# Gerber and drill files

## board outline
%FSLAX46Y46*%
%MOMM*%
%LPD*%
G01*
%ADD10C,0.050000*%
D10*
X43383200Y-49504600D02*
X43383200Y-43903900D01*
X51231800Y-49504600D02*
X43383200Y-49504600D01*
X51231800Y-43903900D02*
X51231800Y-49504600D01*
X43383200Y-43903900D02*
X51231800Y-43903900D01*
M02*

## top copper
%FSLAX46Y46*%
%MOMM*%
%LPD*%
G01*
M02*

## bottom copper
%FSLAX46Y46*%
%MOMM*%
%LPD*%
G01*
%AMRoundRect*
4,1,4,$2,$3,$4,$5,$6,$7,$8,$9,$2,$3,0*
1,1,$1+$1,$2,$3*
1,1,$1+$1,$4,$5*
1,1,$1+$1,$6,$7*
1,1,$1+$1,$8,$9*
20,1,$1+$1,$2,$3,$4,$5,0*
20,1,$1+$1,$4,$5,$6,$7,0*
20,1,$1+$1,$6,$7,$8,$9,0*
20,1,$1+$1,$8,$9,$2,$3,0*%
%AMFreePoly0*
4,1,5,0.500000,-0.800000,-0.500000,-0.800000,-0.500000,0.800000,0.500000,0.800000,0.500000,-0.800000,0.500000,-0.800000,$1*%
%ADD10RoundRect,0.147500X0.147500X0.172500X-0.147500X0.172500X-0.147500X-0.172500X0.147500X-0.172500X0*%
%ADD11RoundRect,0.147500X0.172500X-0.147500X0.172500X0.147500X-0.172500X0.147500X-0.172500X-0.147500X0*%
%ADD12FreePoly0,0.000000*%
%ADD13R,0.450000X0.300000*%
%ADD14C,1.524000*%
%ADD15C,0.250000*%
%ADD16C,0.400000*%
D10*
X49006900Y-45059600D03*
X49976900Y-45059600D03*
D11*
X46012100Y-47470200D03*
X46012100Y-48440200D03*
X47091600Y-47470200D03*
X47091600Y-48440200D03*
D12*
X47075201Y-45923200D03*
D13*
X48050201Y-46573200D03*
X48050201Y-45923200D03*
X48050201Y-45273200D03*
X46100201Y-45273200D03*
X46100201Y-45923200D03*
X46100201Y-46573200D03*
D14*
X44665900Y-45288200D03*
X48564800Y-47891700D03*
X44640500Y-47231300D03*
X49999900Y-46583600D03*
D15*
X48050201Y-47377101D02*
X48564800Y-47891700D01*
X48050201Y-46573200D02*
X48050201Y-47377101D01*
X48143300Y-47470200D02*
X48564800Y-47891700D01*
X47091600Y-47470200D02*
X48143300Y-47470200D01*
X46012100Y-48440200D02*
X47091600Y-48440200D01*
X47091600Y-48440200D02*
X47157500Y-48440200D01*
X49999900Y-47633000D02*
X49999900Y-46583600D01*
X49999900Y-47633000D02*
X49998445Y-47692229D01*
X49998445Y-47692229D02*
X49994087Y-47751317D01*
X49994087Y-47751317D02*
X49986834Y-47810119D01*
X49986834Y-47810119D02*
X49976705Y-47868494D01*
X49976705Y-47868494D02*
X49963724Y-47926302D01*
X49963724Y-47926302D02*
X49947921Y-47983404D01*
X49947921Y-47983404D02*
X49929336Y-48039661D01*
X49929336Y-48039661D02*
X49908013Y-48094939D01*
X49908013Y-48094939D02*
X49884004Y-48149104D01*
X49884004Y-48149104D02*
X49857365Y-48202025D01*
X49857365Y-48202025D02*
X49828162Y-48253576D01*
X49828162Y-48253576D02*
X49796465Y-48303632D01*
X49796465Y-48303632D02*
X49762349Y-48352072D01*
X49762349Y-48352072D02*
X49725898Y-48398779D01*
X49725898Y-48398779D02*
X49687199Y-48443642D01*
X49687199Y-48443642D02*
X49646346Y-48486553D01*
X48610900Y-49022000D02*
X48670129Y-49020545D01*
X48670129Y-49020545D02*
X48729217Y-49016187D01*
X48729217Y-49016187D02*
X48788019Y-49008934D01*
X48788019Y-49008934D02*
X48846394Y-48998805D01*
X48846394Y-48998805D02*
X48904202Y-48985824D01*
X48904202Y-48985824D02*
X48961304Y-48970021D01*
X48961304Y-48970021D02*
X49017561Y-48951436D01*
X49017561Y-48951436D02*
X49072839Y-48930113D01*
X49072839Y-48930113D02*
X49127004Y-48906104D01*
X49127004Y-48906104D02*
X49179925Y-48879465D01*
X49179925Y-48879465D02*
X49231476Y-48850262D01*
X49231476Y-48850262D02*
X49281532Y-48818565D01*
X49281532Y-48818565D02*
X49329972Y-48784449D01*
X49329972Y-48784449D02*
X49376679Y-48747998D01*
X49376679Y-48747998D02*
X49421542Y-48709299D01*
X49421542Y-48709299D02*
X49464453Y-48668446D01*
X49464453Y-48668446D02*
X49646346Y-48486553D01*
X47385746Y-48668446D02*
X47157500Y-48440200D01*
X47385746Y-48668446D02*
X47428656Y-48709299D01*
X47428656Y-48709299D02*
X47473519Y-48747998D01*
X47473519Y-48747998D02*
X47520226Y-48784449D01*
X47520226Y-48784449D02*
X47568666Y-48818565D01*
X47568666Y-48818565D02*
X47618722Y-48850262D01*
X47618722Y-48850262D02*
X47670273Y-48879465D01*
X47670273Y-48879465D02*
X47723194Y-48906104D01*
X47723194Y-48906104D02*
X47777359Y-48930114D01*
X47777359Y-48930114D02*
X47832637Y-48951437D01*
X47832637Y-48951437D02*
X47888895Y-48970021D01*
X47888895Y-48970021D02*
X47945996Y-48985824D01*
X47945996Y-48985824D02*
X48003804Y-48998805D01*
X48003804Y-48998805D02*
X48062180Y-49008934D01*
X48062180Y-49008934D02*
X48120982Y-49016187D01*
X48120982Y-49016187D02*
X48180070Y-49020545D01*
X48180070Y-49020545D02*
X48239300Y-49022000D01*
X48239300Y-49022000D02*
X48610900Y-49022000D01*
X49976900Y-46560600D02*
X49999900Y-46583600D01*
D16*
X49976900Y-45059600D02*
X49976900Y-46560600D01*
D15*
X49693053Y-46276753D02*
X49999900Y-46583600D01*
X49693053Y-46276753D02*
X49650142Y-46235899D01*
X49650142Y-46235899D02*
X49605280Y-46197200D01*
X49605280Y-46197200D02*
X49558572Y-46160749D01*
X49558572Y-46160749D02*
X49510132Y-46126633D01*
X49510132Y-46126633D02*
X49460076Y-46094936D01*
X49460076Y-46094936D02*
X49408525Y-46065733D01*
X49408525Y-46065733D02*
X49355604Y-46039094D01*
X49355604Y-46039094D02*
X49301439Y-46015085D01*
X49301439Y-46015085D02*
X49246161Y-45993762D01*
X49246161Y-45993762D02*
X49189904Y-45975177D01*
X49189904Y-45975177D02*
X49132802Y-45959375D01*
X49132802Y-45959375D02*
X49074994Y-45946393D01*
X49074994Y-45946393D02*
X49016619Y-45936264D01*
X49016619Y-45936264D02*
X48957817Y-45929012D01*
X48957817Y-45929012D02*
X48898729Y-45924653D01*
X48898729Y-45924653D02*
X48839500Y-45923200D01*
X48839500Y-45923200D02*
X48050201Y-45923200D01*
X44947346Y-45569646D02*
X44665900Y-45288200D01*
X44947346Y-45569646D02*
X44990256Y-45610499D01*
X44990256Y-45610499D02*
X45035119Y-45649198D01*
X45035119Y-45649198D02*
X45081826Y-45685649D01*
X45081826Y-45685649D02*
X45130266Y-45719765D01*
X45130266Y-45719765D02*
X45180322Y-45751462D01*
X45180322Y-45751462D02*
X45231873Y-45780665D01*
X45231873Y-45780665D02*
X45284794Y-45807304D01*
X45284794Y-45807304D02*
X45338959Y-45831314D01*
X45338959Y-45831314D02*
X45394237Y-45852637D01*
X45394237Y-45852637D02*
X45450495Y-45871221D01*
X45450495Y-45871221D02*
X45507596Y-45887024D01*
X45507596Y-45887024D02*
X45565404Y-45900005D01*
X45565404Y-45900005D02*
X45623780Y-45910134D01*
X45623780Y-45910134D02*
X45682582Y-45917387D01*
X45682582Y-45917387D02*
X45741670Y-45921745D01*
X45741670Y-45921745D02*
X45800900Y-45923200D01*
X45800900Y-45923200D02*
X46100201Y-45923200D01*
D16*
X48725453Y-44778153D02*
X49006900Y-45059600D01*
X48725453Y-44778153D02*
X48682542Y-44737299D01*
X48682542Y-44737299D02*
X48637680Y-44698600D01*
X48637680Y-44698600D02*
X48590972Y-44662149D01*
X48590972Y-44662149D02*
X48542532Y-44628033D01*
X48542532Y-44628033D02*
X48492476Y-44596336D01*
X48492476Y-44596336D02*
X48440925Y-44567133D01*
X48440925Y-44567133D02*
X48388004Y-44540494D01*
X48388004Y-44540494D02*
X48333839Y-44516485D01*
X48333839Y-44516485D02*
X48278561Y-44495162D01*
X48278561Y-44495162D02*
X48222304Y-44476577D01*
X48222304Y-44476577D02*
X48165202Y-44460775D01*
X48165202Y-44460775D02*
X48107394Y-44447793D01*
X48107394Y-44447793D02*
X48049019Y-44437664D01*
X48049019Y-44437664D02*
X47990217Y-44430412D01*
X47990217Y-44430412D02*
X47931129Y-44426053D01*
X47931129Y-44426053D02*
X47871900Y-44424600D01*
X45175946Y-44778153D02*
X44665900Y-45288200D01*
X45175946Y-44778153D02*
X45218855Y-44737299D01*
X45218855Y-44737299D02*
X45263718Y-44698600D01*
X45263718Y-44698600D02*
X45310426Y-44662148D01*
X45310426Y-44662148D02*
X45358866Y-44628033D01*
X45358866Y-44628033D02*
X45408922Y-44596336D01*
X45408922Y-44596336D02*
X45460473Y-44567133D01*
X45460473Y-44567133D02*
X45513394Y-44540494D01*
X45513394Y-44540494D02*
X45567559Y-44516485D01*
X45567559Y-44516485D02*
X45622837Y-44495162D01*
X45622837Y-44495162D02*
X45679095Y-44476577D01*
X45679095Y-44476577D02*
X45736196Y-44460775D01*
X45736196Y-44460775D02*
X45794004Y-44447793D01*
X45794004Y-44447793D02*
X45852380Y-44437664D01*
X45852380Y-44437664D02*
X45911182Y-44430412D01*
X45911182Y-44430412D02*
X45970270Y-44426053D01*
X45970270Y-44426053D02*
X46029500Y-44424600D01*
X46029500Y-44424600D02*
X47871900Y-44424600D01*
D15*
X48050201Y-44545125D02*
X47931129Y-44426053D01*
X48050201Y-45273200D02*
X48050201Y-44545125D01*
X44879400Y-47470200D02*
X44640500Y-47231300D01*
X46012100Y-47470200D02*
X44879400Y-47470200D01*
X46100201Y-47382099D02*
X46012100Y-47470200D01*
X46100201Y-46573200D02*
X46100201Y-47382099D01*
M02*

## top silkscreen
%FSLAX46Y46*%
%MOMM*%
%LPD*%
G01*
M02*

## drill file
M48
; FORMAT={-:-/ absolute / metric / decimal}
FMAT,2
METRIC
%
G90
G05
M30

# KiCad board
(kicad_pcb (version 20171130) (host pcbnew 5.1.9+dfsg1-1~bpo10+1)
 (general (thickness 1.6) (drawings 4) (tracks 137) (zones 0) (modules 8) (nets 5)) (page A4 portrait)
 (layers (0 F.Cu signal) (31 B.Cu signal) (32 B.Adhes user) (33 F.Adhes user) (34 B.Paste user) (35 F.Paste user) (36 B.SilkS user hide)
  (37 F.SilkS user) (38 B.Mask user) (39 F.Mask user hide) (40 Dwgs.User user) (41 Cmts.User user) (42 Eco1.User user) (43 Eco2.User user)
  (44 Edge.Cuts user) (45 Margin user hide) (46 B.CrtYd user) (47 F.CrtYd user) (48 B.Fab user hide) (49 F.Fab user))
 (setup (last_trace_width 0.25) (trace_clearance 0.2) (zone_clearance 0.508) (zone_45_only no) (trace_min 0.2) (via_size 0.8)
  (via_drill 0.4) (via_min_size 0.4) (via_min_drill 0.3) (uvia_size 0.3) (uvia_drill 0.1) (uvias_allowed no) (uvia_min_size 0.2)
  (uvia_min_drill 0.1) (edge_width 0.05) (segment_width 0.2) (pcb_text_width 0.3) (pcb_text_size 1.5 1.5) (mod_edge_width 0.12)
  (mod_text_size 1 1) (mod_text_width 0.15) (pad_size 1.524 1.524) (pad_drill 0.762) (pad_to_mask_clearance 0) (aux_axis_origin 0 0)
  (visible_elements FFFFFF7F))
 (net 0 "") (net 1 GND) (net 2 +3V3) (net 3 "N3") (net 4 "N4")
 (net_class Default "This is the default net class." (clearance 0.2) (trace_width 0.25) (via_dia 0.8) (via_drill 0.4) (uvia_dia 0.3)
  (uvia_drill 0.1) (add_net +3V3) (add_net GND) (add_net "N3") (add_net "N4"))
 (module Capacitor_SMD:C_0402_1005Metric (layer B.Cu) (at 49.4919 45.0596 180)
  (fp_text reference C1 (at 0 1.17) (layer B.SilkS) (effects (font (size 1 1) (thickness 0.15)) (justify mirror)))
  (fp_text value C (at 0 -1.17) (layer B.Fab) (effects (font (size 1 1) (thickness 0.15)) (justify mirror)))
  (pad 2 smd roundrect (at 0.485 0 180) (size 0.59 0.64) (layers B.Cu B.Paste B.Mask) (roundrect_rratio 0.25) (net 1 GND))
  (pad 1 smd roundrect (at -0.485 0 180) (size 0.59 0.64) (layers B.Cu B.Paste B.Mask) (roundrect_rratio 0.25) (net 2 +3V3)))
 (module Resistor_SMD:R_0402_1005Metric (layer B.Cu) (at 46.0121 47.9552 90)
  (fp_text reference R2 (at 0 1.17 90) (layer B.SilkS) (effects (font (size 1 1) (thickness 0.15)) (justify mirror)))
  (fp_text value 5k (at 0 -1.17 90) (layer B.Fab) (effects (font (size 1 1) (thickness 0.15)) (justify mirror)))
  (pad 2 smd roundrect (at 0.485 0 90) (size 0.59 0.64) (layers B.Cu B.Paste B.Mask) (roundrect_rratio 0.25) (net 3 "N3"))
  (pad 1 smd roundrect (at -0.485 0 90) (size 0.59 0.64) (layers B.Cu B.Paste B.Mask) (roundrect_rratio 0.25) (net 2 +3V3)))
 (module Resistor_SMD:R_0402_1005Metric (layer B.Cu) (at 47.0916 47.9552 90)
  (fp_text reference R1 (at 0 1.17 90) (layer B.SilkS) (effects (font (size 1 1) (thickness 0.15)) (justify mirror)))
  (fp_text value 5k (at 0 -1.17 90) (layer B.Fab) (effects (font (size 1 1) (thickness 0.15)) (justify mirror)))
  (pad 2 smd roundrect (at 0.485 0 90) (size 0.59 0.64) (layers B.Cu B.Paste B.Mask) (roundrect_rratio 0.25) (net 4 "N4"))
  (pad 1 smd roundrect (at -0.485 0 90) (size 0.59 0.64) (layers B.Cu B.Paste B.Mask) (roundrect_rratio 0.25) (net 2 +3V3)))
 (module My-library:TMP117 (layer B.Cu) (at 47.075201 45.9232)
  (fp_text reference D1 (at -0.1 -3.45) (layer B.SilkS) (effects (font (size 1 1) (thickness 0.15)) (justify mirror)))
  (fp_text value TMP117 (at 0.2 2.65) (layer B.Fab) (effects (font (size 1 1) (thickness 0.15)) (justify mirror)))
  (pad 7 smd custom (at 0 0) (size 1 1.6) (layers B.Cu B.Paste B.Mask) (zone_connect 0) (options (clearance outline) (anchor rect))
   (primitives))
  (pad 6 smd rect (at 0.975 0.65) (size 0.45 0.3) (layers B.Cu B.Paste B.Mask) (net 4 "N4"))
  (pad 5 smd rect (at 0.975 0) (size 0.45 0.3) (layers B.Cu B.Paste B.Mask) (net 2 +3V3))
  (pad 4 smd rect (at 0.975 -0.65) (size 0.45 0.3) (layers B.Cu B.Paste B.Mask) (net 1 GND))
  (pad 3 smd rect (at -0.975 -0.65) (size 0.45 0.3) (layers B.Cu B.Paste B.Mask))
  (pad 2 smd rect (at -0.975 0) (size 0.45 0.3) (layers B.Cu B.Paste B.Mask) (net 1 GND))
  (pad 1 smd rect (at -0.975 0.65) (size 0.45 0.3) (layers B.Cu B.Paste B.Mask) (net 3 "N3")))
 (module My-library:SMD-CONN (layer B.Cu) (at 44.6659 45.2882)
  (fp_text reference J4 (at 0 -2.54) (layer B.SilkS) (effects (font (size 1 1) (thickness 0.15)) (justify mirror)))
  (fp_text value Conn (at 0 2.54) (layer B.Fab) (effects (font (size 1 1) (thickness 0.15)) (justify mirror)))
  (pad 1 smd circle (at 0 0) (size 1.524 1.524) (layers B.Cu B.Paste B.Mask) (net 1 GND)))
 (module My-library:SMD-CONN (layer B.Cu) (at 48.5648 47.8917)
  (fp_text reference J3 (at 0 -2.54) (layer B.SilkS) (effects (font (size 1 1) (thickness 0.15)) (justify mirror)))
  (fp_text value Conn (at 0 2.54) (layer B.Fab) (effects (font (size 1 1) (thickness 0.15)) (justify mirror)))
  (pad 1 smd circle (at 0 0) (size 1.524 1.524) (layers B.Cu B.Paste B.Mask) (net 4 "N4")))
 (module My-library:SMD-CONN (layer B.Cu) (at 44.6405 47.2313)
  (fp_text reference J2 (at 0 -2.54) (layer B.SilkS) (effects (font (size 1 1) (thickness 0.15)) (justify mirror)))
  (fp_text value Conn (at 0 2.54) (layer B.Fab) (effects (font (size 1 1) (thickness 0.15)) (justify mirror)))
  (pad 1 smd circle (at 0 0) (size 1.524 1.524) (layers B.Cu B.Paste B.Mask) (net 3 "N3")))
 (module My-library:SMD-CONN (layer B.Cu) (at 49.9999 46.5836)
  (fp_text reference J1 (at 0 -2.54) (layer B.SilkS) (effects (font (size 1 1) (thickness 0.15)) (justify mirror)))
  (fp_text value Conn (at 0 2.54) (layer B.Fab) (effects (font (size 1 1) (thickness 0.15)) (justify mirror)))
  (pad 1 smd circle (at 0 0) (size 1.524 1.524) (layers B.Cu B.Paste B.Mask) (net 2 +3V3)))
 (gr_line (start 43.3832 49.5046) (end 43.3832 43.9039) (layer Edge.Cuts) (width 0.05))
 (gr_line (start 51.2318 49.5046) (end 43.3832 49.5046) (layer Edge.Cuts) (width 0.05))
 (gr_line (start 51.2318 43.9039) (end 51.2318 49.5046) (layer Edge.Cuts) (width 0.05))
 (gr_line (start 43.3832 43.9039) (end 51.2318 43.9039) (layer Edge.Cuts) (width 0.05))
 (segment (start 48.050201 47.377101) (end 48.5648 47.8917) (width 0.25) (layer B.Cu) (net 4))
 (segment (start 48.050201 46.5732) (end 48.050201 47.377101) (width 0.25) (layer B.Cu) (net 4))
 (segment (start 48.1433 47.4702) (end 48.5648 47.8917) (width 0.25) (layer B.Cu) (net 4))
 (segment (start 47.0916 47.4702) (end 48.1433 47.4702) (width 0.25) (layer B.Cu) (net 4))
 (segment (start 46.0121 48.4402) (end 47.0916 48.4402) (width 0.25) (layer B.Cu) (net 2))
 (segment (start 47.0916 48.4402) (end 47.1575 48.4402) (width 0.25) (layer B.Cu) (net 2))
 (segment (start 49.9999 47.633) (end 49.9999 46.5836) (width 0.25) (layer B.Cu) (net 2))
 (segment (start 49.9999 47.633) (end 49.998445 47.692229) (width 0.25) (layer B.Cu) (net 2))
 (segment (start 49.998445 47.692229) (end 49.994087 47.751317) (width 0.25) (layer B.Cu) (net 2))
 (segment (start 49.994087 47.751317) (end 49.986834 47.810119) (width 0.25) (layer B.Cu) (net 2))
 (segment (start 49.986834 47.810119) (end 49.976705 47.868494) (width 0.25) (layer B.Cu) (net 2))
 (segment (start 49.976705 47.868494) (end 49.963724 47.926302) (width 0.25) (layer B.Cu) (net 2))
 (segment (start 49.963724 47.926302) (end 49.947921 47.983404) (width 0.25) (layer B.Cu) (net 2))
 (segment (start 49.947921 47.983404) (end 49.929336 48.039661) (width 0.25) (layer B.Cu) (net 2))
 (segment (start 49.929336 48.039661) (end 49.908013 48.094939) (width 0.25) (layer B.Cu) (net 2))
 (segment (start 49.908013 48.094939) (end 49.884004 48.149104) (width 0.25) (layer B.Cu) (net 2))
 (segment (start 49.884004 48.149104) (end 49.857365 48.202025) (width 0.25) (layer B.Cu) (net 2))
 (segment (start 49.857365 48.202025) (end 49.828162 48.253576) (width 0.25) (layer B.Cu) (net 2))
 (segment (start 49.828162 48.253576) (end 49.796465 48.303632) (width 0.25) (layer B.Cu) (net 2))
 (segment (start 49.796465 48.303632) (end 49.762349 48.352072) (width 0.25) (layer B.Cu) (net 2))
 (segment (start 49.762349 48.352072) (end 49.725898 48.398779) (width 0.25) (layer B.Cu) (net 2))
 (segment (start 49.725898 48.398779) (end 49.687199 48.443642) (width 0.25) (layer B.Cu) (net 2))
 (segment (start 49.687199 48.443642) (end 49.646346 48.486553) (width 0.25) (layer B.Cu) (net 2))
 (segment (start 48.6109 49.022) (end 48.670129 49.020545) (width 0.25) (layer B.Cu) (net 2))
 (segment (start 48.670129 49.020545) (end 48.729217 49.016187) (width 0.25) (layer B.Cu) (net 2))
 (segment (start 48.729217 49.016187) (end 48.788019 49.008934) (width 0.25) (layer B.Cu) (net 2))
 (segment (start 48.788019 49.008934) (end 48.846394 48.998805) (width 0.25) (layer B.Cu) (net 2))
 (segment (start 48.846394 48.998805) (end 48.904202 48.985824) (width 0.25) (layer B.Cu) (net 2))
 (segment (start 48.904202 48.985824) (end 48.961304 48.970021) (width 0.25) (layer B.Cu) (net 2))
 (segment (start 48.961304 48.970021) (end 49.017561 48.951436) (width 0.25) (layer B.Cu) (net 2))
 (segment (start 49.017561 48.951436) (end 49.072839 48.930113) (width 0.25) (layer B.Cu) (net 2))
 (segment (start 49.072839 48.930113) (end 49.127004 48.906104) (width 0.25) (layer B.Cu) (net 2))
 (segment (start 49.127004 48.906104) (end 49.179925 48.879465) (width 0.25) (layer B.Cu) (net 2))
 (segment (start 49.179925 48.879465) (end 49.231476 48.850262) (width 0.25) (layer B.Cu) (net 2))
 (segment (start 49.231476 48.850262) (end 49.281532 48.818565) (width 0.25) (layer B.Cu) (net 2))
 (segment (start 49.281532 48.818565) (end 49.329972 48.784449) (width 0.25) (layer B.Cu) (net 2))
 (segment (start 49.329972 48.784449) (end 49.376679 48.747998) (width 0.25) (layer B.Cu) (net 2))
 (segment (start 49.376679 48.747998) (end 49.421542 48.709299) (width 0.25) (layer B.Cu) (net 2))
 (segment (start 49.421542 48.709299) (end 49.464453 48.668446) (width 0.25) (layer B.Cu) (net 2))
 (segment (start 49.464453 48.668446) (end 49.646346 48.486553) (width 0.25) (layer B.Cu) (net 2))
 (segment (start 47.385746 48.668446) (end 47.1575 48.4402) (width 0.25) (layer B.Cu) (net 2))
 (segment (start 47.385746 48.668446) (end 47.428656 48.709299) (width 0.25) (layer B.Cu) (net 2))
 (segment (start 47.428656 48.709299) (end 47.473519 48.747998) (width 0.25) (layer B.Cu) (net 2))
 (segment (start 47.473519 48.747998) (end 47.520226 48.784449) (width 0.25) (layer B.Cu) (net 2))
 (segment (start 47.520226 48.784449) (end 47.568666 48.818565) (width 0.25) (layer B.Cu) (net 2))
 (segment (start 47.568666 48.818565) (end 47.618722 48.850262) (width 0.25) (layer B.Cu) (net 2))
 (segment (start 47.618722 48.850262) (end 47.670273 48.879465) (width 0.25) (layer B.Cu) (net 2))
 (segment (start 47.670273 48.879465) (end 47.723194 48.906104) (width 0.25) (layer B.Cu) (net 2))
 (segment (start 47.723194 48.906104) (end 47.777359 48.930114) (width 0.25) (layer B.Cu) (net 2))
 (segment (start 47.777359 48.930114) (end 47.832637 48.951437) (width 0.25) (layer B.Cu) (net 2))
 (segment (start 47.832637 48.951437) (end 47.888895 48.970021) (width 0.25) (layer B.Cu) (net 2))
 (segment (start 47.888895 48.970021) (end 47.945996 48.985824) (width 0.25) (layer B.Cu) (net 2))
 (segment (start 47.945996 48.985824) (end 48.003804 48.998805) (width 0.25) (layer B.Cu) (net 2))
 (segment (start 48.003804 48.998805) (end 48.06218 49.008934) (width 0.25) (layer B.Cu) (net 2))
 (segment (start 48.06218 49.008934) (end 48.120982 49.016187) (width 0.25) (layer B.Cu) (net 2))
 (segment (start 48.120982 49.016187) (end 48.18007 49.020545) (width 0.25) (layer B.Cu) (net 2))
 (segment (start 48.18007 49.020545) (end 48.2393 49.022) (width 0.25) (layer B.Cu) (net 2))
 (segment (start 48.2393 49.022) (end 48.6109 49.022) (width 0.25) (layer B.Cu) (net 2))
 (segment (start 49.9769 46.5606) (end 49.9999 46.5836) (width 0.25) (layer B.Cu) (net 2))
 (segment (start 49.9769 45.0596) (end 49.9769 46.5606) (width 0.4) (layer B.Cu) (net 2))
 (segment (start 49.693053 46.276753) (end 49.9999 46.5836) (width 0.25) (layer B.Cu) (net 2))
 (segment (start 49.693053 46.276753) (end 49.650142 46.235899) (width 0.25) (layer B.Cu) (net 2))
 (segment (start 49.650142 46.235899) (end 49.60528 46.1972) (width 0.25) (layer B.Cu) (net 2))
 (segment (start 49.60528 46.1972) (end 49.558572 46.160749) (width 0.25) (layer B.Cu) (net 2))
 (segment (start 49.558572 46.160749) (end 49.510132 46.126633) (width 0.25) (layer B.Cu) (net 2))
 (segment (start 49.510132 46.126633) (end 49.460076 46.094936) (width 0.25) (layer B.Cu) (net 2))
 (segment (start 49.460076 46.094936) (end 49.408525 46.065733) (width 0.25) (layer B.Cu) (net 2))
 (segment (start 49.408525 46.065733) (end 49.355604 46.039094) (width 0.25) (layer B.Cu) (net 2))
 (segment (start 49.355604 46.039094) (end 49.301439 46.015085) (width 0.25) (layer B.Cu) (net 2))
 (segment (start 49.301439 46.015085) (end 49.246161 45.993762) (width 0.25) (layer B.Cu) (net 2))
 (segment (start 49.246161 45.993762) (end 49.189904 45.975177) (width 0.25) (layer B.Cu) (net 2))
 (segment (start 49.189904 45.975177) (end 49.132802 45.959375) (width 0.25) (layer B.Cu) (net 2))
 (segment (start 49.132802 45.959375) (end 49.074994 45.946393) (width 0.25) (layer B.Cu) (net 2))
 (segment (start 49.074994 45.946393) (end 49.016619 45.936264) (width 0.25) (layer B.Cu) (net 2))
 (segment (start 49.016619 45.936264) (end 48.957817 45.929012) (width 0.25) (layer B.Cu) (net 2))
 (segment (start 48.957817 45.929012) (end 48.898729 45.924653) (width 0.25) (layer B.Cu) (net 2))
 (segment (start 48.898729 45.924653) (end 48.8395 45.9232) (width 0.25) (layer B.Cu) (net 2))
 (segment (start 48.8395 45.9232) (end 48.050201 45.9232) (width 0.25) (layer B.Cu) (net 2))
 (segment (start 44.947346 45.569646) (end 44.6659 45.2882) (width 0.25) (layer B.Cu) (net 1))
 (segment (start 44.947346 45.569646) (end 44.990256 45.610499) (width 0.25) (layer B.Cu) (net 1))
 (segment (start 44.990256 45.610499) (end 45.035119 45.649198) (width 0.25) (layer B.Cu) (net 1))
 (segment (start 45.035119 45.649198) (end 45.081826 45.685649) (width 0.25) (layer B.Cu) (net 1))
 (segment (start 45.081826 45.685649) (end 45.130266 45.719765) (width 0.25) (layer B.Cu) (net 1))
 (segment (start 45.130266 45.719765) (end 45.180322 45.751462) (width 0.25) (layer B.Cu) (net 1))
 (segment (start 45.180322 45.751462) (end 45.231873 45.780665) (width 0.25) (layer B.Cu) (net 1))
 (segment (start 45.231873 45.780665) (end 45.284794 45.807304) (width 0.25) (layer B.Cu) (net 1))
 (segment (start 45.284794 45.807304) (end 45.338959 45.831314) (width 0.25) (layer B.Cu) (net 1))
 (segment (start 45.338959 45.831314) (end 45.394237 45.852637) (width 0.25) (layer B.Cu) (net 1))
 (segment (start 45.394237 45.852637) (end 45.450495 45.871221) (width 0.25) (layer B.Cu) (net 1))
 (segment (start 45.450495 45.871221) (end 45.507596 45.887024) (width 0.25) (layer B.Cu) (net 1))
 (segment (start 45.507596 45.887024) (end 45.565404 45.900005) (width 0.25) (layer B.Cu) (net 1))
 (segment (start 45.565404 45.900005) (end 45.62378 45.910134) (width 0.25) (layer B.Cu) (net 1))
 (segment (start 45.62378 45.910134) (end 45.682582 45.917387) (width 0.25) (layer B.Cu) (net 1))
 (segment (start 45.682582 45.917387) (end 45.74167 45.921745) (width 0.25) (layer B.Cu) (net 1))
 (segment (start 45.74167 45.921745) (end 45.8009 45.9232) (width 0.25) (layer B.Cu) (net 1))
 (segment (start 45.8009 45.9232) (end 46.100201 45.9232) (width 0.25) (layer B.Cu) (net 1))
 (segment (start 48.725453 44.778153) (end 49.0069 45.0596) (width 0.4) (layer B.Cu) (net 1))
 (segment (start 48.725453 44.778153) (end 48.682542 44.737299) (width 0.4) (layer B.Cu) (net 1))
 (segment (start 48.682542 44.737299) (end 48.63768 44.6986) (width 0.4) (layer B.Cu) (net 1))
 (segment (start 48.63768 44.6986) (end 48.590972 44.662149) (width 0.4) (layer B.Cu) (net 1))
 (segment (start 48.590972 44.662149) (end 48.542532 44.628033) (width 0.4) (layer B.Cu) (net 1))
 (segment (start 48.542532 44.628033) (end 48.492476 44.596336) (width 0.4) (layer B.Cu) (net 1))
 (segment (start 48.492476 44.596336) (end 48.440925 44.567133) (width 0.4) (layer B.Cu) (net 1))
 (segment (start 48.440925 44.567133) (end 48.388004 44.540494) (width 0.4) (layer B.Cu) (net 1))
 (segment (start 48.388004 44.540494) (end 48.333839 44.516485) (width 0.4) (layer B.Cu) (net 1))
 (segment (start 48.333839 44.516485) (end 48.278561 44.495162) (width 0.4) (layer B.Cu) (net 1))
 (segment (start 48.278561 44.495162) (end 48.222304 44.476577) (width 0.4) (layer B.Cu) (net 1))
 (segment (start 48.222304 44.476577) (end 48.165202 44.460775) (width 0.4) (layer B.Cu) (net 1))
 (segment (start 48.165202 44.460775) (end 48.107394 44.447793) (width 0.4) (layer B.Cu) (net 1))
 (segment (start 48.107394 44.447793) (end 48.049019 44.437664) (width 0.4) (layer B.Cu) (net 1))
 (segment (start 48.049019 44.437664) (end 47.990217 44.430412) (width 0.4) (layer B.Cu) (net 1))
 (segment (start 47.990217 44.430412) (end 47.931129 44.426053) (width 0.4) (layer B.Cu) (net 1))
 (segment (start 47.931129 44.426053) (end 47.8719 44.4246) (width 0.4) (layer B.Cu) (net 1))
 (segment (start 45.175946 44.778153) (end 44.6659 45.2882) (width 0.4) (layer B.Cu) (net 1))
 (segment (start 45.175946 44.778153) (end 45.218855 44.737299) (width 0.4) (layer B.Cu) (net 1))
 (segment (start 45.218855 44.737299) (end 45.263718 44.6986) (width 0.4) (layer B.Cu) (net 1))
 (segment (start 45.263718 44.6986) (end 45.310426 44.662148) (width 0.4) (layer B.Cu) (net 1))
 (segment (start 45.310426 44.662148) (end 45.358866 44.628033) (width 0.4) (layer B.Cu) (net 1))
 (segment (start 45.358866 44.628033) (end 45.408922 44.596336) (width 0.4) (layer B.Cu) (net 1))
 (segment (start 45.408922 44.596336) (end 45.460473 44.567133) (width 0.4) (layer B.Cu) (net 1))
 (segment (start 45.460473 44.567133) (end 45.513394 44.540494) (width 0.4) (layer B.Cu) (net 1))
 (segment (start 45.513394 44.540494) (end 45.567559 44.516485) (width 0.4) (layer B.Cu) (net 1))
 (segment (start 45.567559 44.516485) (end 45.622837 44.495162) (width 0.4) (layer B.Cu) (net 1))
 (segment (start 45.622837 44.495162) (end 45.679095 44.476577) (width 0.4) (layer B.Cu) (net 1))
 (segment (start 45.679095 44.476577) (end 45.736196 44.460775) (width 0.4) (layer B.Cu) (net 1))
 (segment (start 45.736196 44.460775) (end 45.794004 44.447793) (width 0.4) (layer B.Cu) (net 1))
 (segment (start 45.794004 44.447793) (end 45.85238 44.437664) (width 0.4) (layer B.Cu) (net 1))
 (segment (start 45.85238 44.437664) (end 45.911182 44.430412) (width 0.4) (layer B.Cu) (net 1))
 (segment (start 45.911182 44.430412) (end 45.97027 44.426053) (width 0.4) (layer B.Cu) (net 1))
 (segment (start 45.97027 44.426053) (end 46.0295 44.4246) (width 0.4) (layer B.Cu) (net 1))
 (segment (start 46.0295 44.4246) (end 47.8719 44.4246) (width 0.4) (layer B.Cu) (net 1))
 (segment (start 48.050201 44.545125) (end 47.931129 44.426053) (width 0.25) (layer B.Cu) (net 1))
 (segment (start 48.050201 45.2732) (end 48.050201 44.545125) (width 0.25) (layer B.Cu) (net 1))
 (segment (start 44.8794 47.4702) (end 44.6405 47.2313) (width 0.25) (layer B.Cu) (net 3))
 (segment (start 46.0121 47.4702) (end 44.8794 47.4702) (width 0.25) (layer B.Cu) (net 3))
 (segment (start 46.100201 47.382099) (end 46.0121 47.4702) (width 0.25) (layer B.Cu) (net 3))
 (segment (start 46.100201 46.5732) (end 46.100201 47.382099) (width 0.25) (layer B.Cu) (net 3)))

